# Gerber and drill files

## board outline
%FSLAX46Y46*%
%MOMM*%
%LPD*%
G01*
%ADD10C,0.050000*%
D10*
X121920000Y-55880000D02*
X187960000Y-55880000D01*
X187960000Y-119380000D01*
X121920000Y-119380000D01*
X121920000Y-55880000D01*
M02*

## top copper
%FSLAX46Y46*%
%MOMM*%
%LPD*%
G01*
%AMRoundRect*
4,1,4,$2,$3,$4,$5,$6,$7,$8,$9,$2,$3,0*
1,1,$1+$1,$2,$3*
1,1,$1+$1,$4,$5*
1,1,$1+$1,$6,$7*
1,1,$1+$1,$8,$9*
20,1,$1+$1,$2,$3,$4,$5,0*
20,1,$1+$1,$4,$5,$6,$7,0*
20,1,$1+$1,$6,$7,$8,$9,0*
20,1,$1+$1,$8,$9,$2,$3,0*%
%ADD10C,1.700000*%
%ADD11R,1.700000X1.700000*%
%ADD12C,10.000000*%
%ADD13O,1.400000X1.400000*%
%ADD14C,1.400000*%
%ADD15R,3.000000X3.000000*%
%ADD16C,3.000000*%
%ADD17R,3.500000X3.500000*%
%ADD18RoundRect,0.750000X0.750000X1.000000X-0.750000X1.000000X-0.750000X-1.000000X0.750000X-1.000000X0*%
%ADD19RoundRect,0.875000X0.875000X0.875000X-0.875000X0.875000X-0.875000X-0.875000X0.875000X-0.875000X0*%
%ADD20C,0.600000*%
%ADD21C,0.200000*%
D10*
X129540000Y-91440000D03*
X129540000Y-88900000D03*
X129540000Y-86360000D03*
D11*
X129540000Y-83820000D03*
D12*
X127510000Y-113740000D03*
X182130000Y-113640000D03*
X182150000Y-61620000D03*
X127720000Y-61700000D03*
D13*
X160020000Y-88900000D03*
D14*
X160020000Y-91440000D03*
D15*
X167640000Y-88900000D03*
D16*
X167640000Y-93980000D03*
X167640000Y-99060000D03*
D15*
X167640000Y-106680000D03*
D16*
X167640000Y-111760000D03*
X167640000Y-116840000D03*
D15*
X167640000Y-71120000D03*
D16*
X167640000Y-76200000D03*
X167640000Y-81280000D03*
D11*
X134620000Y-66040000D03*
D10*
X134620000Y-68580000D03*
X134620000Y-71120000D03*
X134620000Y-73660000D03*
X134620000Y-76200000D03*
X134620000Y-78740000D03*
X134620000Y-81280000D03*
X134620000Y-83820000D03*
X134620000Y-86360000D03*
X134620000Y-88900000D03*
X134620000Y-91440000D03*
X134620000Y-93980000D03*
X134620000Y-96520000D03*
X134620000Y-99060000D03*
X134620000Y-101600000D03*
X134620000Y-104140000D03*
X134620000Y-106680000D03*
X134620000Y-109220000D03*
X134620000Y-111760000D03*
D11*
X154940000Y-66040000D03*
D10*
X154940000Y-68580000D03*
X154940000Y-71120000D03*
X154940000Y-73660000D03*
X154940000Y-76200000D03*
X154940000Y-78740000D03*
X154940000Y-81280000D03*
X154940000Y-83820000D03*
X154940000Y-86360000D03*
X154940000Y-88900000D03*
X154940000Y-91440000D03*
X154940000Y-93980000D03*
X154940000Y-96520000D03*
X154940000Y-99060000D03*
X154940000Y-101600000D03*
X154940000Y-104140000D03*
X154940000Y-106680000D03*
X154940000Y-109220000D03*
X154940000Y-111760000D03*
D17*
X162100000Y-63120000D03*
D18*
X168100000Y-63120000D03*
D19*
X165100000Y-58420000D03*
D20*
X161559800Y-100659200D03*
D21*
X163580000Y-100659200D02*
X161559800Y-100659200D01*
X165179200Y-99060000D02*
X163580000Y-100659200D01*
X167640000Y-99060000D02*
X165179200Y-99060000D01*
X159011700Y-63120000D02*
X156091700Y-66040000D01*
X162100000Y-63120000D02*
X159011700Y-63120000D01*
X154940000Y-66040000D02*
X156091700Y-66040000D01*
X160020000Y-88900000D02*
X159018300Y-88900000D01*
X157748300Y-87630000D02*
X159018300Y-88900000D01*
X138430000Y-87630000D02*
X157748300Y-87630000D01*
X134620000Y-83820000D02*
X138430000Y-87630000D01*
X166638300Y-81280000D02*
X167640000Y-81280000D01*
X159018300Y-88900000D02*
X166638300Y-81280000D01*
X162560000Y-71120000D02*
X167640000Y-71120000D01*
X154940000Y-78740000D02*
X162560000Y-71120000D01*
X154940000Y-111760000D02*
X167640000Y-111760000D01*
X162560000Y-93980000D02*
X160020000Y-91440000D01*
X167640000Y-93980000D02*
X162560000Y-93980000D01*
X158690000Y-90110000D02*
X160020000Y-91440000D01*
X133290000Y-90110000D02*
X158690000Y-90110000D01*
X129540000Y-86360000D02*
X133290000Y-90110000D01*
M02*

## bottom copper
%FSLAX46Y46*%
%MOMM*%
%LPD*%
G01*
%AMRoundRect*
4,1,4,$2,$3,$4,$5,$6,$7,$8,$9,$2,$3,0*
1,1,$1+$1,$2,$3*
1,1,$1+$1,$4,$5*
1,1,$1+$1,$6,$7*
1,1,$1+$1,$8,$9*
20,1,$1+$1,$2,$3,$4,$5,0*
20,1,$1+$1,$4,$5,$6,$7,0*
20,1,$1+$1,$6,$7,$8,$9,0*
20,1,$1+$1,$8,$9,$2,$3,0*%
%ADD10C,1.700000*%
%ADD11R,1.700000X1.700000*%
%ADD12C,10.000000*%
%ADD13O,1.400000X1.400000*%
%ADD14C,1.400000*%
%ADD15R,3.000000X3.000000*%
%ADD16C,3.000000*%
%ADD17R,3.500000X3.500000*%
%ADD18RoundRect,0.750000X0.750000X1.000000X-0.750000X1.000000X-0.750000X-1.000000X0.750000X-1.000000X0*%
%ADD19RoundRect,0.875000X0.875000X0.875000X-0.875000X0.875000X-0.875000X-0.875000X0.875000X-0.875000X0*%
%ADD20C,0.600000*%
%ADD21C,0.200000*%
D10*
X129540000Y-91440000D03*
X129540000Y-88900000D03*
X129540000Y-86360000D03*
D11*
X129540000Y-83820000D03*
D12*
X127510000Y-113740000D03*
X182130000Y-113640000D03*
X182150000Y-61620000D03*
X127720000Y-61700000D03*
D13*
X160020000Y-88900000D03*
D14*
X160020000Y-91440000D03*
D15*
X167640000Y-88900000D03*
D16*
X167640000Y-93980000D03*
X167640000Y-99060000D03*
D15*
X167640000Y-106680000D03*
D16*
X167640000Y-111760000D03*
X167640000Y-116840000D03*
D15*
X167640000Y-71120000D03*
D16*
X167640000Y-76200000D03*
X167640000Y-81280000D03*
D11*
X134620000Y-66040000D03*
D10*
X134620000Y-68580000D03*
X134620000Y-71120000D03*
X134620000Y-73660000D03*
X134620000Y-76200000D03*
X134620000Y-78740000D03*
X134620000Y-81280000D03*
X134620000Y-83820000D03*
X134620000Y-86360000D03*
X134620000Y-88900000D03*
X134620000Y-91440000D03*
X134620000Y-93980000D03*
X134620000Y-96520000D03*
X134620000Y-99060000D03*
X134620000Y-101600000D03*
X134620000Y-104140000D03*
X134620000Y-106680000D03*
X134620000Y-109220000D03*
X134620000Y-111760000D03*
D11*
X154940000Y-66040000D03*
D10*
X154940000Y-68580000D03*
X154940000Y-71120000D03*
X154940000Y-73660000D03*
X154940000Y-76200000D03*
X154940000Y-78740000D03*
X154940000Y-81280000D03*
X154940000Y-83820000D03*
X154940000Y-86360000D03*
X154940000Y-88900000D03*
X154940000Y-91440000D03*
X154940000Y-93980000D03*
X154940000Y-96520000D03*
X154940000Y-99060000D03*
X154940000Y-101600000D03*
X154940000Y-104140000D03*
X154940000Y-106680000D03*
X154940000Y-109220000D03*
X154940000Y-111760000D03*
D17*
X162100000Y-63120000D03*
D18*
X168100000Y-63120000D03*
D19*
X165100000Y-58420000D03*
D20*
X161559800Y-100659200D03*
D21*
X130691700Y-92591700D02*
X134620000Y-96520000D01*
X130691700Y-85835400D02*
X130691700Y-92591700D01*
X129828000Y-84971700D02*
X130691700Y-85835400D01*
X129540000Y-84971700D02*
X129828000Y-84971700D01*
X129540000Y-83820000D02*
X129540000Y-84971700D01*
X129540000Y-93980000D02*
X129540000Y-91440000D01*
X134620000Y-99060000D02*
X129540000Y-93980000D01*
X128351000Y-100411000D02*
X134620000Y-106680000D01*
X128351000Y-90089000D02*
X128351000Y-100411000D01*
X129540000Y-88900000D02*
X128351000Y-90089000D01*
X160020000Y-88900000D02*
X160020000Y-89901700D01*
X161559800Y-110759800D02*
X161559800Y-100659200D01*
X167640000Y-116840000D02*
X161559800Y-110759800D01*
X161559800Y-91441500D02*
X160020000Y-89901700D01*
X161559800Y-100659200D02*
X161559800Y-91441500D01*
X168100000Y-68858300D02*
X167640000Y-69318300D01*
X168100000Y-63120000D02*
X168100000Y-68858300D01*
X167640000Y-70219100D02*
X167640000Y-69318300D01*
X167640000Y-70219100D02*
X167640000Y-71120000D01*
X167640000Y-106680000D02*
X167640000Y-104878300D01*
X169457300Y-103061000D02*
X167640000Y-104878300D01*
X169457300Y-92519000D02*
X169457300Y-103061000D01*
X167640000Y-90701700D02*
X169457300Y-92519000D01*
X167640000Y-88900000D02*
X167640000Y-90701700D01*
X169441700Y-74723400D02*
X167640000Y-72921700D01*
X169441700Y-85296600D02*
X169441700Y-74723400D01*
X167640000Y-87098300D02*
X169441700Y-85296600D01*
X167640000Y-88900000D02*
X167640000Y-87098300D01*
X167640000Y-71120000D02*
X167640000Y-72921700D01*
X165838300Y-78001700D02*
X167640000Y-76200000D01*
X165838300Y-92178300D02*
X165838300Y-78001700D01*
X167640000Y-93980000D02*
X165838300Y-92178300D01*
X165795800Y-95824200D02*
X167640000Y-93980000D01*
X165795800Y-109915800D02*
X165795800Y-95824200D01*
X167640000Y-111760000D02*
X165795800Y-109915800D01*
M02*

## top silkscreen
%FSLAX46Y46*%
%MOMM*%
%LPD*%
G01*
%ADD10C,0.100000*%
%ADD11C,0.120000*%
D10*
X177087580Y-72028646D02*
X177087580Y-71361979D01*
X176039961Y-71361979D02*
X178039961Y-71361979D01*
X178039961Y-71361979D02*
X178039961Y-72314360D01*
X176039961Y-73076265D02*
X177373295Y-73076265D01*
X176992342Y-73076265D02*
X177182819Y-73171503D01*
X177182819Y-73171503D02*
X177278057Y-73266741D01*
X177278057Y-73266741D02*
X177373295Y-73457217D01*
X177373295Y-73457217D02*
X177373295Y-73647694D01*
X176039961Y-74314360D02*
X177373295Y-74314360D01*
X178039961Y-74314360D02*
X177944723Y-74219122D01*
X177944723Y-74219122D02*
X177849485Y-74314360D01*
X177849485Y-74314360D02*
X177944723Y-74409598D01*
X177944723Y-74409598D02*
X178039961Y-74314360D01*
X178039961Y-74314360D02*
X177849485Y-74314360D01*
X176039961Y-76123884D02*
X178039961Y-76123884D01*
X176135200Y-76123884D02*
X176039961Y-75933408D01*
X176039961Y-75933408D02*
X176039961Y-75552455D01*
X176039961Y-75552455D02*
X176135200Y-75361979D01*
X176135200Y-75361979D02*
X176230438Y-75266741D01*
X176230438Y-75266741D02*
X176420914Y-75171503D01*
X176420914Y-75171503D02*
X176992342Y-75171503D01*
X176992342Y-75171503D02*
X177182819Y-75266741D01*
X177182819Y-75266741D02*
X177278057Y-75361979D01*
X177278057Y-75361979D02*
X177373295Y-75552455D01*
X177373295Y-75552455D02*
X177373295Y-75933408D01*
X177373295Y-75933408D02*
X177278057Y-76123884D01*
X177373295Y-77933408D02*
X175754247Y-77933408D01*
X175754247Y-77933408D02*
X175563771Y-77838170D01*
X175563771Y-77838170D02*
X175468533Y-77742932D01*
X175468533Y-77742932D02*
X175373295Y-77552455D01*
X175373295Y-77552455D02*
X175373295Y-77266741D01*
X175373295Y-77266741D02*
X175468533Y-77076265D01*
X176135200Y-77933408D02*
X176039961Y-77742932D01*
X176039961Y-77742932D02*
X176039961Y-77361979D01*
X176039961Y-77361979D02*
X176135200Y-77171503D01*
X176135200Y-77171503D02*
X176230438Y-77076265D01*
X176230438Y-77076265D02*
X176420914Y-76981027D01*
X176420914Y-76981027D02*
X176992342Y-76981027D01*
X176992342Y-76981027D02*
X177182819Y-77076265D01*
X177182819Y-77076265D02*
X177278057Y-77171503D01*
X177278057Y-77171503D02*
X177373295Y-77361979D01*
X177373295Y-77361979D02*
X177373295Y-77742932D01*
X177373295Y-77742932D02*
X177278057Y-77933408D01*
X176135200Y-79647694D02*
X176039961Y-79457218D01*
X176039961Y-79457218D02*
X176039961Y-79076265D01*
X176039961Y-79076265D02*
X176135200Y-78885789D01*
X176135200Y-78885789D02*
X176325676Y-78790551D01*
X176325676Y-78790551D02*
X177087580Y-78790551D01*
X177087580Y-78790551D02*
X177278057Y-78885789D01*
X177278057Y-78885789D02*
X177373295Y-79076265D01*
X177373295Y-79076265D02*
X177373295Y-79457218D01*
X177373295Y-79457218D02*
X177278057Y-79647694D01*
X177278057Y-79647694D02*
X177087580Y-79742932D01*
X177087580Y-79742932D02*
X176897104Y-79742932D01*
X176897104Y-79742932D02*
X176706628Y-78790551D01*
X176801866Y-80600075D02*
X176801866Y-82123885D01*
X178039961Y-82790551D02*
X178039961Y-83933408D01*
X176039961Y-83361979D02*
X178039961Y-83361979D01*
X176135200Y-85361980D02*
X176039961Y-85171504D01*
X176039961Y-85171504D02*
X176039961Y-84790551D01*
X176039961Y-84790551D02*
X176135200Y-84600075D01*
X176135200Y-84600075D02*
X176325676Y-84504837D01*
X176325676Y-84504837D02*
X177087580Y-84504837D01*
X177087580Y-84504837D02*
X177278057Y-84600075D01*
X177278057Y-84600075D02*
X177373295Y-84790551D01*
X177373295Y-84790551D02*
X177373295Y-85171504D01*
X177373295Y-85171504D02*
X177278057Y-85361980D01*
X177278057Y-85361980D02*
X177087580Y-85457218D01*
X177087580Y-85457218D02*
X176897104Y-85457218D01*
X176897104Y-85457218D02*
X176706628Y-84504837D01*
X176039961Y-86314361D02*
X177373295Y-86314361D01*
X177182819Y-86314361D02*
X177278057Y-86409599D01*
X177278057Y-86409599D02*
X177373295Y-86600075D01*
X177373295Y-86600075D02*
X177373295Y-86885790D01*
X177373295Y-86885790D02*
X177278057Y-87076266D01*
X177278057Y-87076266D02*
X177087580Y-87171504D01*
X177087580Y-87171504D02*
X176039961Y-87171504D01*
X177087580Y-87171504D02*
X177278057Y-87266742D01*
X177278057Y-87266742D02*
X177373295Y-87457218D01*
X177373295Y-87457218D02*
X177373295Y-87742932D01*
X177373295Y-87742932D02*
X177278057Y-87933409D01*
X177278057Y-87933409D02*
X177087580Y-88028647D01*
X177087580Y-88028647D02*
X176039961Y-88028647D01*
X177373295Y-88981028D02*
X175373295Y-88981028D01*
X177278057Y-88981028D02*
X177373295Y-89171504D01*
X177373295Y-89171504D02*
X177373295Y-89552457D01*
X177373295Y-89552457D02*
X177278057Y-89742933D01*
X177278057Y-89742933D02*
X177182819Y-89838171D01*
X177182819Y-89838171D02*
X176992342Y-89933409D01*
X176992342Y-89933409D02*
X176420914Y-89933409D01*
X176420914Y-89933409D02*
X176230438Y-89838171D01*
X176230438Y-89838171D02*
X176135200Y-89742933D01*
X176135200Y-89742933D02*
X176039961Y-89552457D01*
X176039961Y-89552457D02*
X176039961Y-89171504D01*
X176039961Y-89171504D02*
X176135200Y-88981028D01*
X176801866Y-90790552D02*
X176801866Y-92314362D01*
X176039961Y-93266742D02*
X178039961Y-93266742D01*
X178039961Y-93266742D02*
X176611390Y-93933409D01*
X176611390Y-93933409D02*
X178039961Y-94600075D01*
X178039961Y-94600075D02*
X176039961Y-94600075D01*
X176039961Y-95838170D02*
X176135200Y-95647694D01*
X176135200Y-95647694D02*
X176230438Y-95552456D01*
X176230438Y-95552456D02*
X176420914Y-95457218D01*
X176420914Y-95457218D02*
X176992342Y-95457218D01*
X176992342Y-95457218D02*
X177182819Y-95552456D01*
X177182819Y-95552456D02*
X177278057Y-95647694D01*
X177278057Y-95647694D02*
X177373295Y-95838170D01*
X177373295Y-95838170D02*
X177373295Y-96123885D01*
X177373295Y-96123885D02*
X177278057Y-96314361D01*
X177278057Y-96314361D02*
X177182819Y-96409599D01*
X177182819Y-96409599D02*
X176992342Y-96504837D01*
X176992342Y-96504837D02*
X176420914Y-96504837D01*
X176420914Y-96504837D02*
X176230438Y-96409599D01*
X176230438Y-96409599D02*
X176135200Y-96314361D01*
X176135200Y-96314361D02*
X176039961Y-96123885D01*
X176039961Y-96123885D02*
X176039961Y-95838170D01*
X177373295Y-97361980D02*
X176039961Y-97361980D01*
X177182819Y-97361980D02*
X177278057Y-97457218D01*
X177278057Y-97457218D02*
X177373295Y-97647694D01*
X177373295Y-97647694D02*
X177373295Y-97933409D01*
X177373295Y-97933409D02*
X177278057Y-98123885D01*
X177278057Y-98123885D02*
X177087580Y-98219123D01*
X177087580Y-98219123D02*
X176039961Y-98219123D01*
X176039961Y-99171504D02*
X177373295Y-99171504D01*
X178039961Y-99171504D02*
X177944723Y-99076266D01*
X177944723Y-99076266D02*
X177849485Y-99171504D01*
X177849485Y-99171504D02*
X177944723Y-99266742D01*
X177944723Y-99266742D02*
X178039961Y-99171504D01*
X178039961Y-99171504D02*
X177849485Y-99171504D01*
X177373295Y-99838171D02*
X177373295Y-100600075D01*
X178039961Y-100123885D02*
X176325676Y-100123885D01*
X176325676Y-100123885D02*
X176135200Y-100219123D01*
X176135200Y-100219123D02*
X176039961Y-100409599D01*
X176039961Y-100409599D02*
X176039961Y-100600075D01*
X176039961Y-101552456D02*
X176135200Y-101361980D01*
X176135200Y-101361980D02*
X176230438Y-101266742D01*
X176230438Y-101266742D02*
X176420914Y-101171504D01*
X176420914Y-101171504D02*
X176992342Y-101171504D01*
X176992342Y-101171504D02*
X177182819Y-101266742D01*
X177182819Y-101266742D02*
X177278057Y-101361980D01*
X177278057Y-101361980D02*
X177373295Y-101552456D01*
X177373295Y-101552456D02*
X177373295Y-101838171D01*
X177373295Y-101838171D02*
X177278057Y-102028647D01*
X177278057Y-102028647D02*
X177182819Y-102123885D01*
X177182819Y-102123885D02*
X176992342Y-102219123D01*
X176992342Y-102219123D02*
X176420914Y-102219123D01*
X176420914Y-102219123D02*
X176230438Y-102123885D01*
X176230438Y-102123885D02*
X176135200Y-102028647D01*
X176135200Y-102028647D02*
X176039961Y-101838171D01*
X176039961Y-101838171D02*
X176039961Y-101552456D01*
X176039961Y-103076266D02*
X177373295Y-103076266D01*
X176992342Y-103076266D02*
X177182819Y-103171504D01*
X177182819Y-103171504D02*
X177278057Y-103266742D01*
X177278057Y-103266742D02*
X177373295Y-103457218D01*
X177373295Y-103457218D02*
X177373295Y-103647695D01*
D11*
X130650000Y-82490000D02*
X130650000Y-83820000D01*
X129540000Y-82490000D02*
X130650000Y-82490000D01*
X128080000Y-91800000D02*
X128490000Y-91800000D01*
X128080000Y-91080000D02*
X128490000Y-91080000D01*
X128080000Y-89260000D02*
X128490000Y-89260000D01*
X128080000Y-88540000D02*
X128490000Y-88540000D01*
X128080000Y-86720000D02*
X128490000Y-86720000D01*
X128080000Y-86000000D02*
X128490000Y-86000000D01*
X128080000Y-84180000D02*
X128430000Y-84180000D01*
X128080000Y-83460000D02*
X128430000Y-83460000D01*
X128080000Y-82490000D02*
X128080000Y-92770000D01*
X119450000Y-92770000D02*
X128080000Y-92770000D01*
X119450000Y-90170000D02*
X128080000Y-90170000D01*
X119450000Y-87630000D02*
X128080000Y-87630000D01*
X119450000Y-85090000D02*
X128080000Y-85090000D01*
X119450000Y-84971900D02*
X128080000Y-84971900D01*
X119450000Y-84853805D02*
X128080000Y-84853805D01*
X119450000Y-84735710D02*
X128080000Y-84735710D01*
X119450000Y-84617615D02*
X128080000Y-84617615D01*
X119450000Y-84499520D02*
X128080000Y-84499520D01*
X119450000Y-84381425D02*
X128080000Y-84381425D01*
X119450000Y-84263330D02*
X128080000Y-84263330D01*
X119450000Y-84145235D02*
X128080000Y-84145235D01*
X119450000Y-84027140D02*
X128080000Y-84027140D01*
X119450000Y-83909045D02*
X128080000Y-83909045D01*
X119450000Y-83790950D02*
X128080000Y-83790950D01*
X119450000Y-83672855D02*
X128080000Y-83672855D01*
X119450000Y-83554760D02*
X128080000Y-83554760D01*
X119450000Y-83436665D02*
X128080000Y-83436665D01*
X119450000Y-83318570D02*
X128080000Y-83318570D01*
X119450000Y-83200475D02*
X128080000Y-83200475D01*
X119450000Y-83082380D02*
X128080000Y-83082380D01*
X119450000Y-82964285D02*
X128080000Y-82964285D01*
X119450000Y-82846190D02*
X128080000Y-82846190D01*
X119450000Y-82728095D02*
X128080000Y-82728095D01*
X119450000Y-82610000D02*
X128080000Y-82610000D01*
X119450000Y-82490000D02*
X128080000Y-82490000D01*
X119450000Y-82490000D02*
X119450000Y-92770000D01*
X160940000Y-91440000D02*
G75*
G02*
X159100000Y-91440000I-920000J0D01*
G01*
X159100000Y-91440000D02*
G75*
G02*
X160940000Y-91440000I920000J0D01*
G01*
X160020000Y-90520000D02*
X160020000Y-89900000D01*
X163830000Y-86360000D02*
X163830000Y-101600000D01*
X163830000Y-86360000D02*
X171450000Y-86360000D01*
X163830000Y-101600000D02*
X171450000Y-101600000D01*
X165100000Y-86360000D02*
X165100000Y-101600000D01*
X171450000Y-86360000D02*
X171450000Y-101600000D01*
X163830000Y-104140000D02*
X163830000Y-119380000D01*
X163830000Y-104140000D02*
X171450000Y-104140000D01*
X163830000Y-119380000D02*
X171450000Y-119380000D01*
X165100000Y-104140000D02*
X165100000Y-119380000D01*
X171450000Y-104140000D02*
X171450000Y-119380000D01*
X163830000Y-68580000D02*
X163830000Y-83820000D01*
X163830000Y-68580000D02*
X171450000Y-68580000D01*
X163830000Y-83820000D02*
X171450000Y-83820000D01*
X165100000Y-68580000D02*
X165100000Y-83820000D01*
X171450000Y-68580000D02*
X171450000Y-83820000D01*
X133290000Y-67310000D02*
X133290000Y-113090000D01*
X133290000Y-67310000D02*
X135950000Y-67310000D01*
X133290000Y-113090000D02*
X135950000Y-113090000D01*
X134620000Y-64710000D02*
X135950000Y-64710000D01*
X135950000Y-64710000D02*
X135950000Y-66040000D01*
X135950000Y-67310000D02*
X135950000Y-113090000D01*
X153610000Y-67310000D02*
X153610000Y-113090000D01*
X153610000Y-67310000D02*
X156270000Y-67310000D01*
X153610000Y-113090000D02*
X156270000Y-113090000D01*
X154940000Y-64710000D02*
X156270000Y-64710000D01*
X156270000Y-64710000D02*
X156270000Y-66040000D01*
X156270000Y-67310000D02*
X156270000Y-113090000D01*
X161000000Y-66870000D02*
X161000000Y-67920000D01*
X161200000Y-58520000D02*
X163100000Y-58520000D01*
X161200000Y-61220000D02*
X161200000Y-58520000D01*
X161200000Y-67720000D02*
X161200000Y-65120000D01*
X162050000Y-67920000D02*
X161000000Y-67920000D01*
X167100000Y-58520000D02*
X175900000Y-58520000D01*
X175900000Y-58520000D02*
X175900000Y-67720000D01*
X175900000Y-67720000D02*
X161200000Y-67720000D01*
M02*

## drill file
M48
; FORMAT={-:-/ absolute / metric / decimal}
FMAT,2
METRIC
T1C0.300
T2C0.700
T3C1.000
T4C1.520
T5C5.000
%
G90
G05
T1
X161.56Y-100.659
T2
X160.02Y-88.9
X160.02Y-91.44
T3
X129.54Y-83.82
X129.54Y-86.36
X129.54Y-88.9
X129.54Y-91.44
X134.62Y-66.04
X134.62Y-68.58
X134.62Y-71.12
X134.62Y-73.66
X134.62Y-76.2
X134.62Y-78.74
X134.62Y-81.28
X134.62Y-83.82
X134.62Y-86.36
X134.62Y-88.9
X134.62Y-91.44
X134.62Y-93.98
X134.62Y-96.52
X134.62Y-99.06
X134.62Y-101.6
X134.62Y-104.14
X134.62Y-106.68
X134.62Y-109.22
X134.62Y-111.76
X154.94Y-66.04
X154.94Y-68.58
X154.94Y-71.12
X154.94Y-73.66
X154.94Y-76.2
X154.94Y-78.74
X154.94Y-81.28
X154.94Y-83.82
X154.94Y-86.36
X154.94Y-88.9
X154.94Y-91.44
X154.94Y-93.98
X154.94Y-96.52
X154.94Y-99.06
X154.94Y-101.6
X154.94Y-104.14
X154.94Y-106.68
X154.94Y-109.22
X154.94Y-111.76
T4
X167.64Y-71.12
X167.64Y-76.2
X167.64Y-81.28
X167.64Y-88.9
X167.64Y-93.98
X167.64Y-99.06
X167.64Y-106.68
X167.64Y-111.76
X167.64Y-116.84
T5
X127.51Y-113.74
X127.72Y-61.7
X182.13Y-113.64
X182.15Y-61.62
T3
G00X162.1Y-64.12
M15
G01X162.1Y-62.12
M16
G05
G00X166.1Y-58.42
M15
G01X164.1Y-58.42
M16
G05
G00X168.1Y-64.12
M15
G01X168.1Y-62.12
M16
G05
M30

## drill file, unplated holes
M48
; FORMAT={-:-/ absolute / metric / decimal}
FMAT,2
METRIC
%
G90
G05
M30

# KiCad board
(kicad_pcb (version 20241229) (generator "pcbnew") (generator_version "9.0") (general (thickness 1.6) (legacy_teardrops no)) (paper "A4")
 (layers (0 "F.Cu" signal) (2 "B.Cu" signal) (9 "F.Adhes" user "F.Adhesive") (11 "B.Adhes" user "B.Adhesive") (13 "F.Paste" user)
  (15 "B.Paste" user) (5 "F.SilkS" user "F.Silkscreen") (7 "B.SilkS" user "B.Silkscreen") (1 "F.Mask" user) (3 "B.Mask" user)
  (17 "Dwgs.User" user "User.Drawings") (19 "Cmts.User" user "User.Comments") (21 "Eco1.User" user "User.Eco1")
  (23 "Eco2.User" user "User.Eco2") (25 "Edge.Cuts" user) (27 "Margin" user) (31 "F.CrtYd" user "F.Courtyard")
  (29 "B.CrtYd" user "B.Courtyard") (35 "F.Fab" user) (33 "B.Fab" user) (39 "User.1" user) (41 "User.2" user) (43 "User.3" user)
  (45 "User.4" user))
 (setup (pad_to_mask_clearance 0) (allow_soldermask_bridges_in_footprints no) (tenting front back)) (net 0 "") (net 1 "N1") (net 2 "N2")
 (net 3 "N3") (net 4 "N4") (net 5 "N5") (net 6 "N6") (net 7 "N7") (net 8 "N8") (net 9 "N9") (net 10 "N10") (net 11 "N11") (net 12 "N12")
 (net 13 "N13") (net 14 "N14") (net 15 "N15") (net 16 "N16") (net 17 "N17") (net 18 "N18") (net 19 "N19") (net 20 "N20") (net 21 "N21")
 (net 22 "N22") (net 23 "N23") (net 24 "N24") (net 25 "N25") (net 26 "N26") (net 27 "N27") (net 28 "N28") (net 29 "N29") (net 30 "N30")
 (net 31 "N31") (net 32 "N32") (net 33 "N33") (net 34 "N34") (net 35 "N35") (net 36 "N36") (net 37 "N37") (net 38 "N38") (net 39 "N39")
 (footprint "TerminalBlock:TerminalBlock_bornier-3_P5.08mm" (layer "F.Cu") (at 167.64 88.9 -90)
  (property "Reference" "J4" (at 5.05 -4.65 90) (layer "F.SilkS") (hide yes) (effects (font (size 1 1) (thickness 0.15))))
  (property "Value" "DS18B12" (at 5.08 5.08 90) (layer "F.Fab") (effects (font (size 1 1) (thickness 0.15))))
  (fp_line (start -2.54 3.81) (end 12.7 3.81) (stroke (width 0.12) (type solid)) (layer "F.SilkS"))
  (fp_line (start -2.54 3.81) (end -2.54 -3.81) (stroke (width 0.12) (type solid)) (layer "F.SilkS"))
  (fp_line (start 12.7 3.81) (end 12.7 -3.81) (stroke (width 0.12) (type solid)) (layer "F.SilkS"))
  (fp_line (start -2.54 2.54) (end 12.7 2.54) (stroke (width 0.12) (type solid)) (layer "F.SilkS"))
  (fp_line (start -2.54 -3.81) (end 12.7 -3.81) (stroke (width 0.12) (type solid)) (layer "F.SilkS"))
  (pad "1" thru_hole rect (at 0 0 270) (size 3 3) (drill 1.52) (layers "*.Cu" "*.Mask") (remove_unused_layers no) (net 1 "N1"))
  (pad "2" thru_hole circle (at 5.08 0 270) (size 3 3) (drill 1.52) (layers "*.Cu" "*.Mask") (remove_unused_layers no) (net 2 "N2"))
  (pad "3" thru_hole circle (at 10.16 0 270) (size 3 3) (drill 1.52) (layers "*.Cu" "*.Mask") (remove_unused_layers no) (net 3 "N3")))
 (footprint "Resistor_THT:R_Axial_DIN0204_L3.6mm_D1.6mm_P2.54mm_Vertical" (layer "F.Cu") (at 160.02 91.44 90)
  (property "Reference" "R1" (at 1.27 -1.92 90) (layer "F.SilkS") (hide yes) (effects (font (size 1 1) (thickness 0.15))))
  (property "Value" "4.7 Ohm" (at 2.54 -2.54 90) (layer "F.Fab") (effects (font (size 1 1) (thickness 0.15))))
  (fp_line (start 0.92 0) (end 1.54 0) (stroke (width 0.12) (type solid)) (layer "F.SilkS"))
  (fp_circle (center 0 0) (end 0.92 0) (stroke (width 0.12) (type solid)) (fill no) (layer "F.SilkS"))
  (pad "1" thru_hole circle (at 0 0 90) (size 1.4 1.4) (drill 0.7) (layers "*.Cu" "*.Mask") (remove_unused_layers no) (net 2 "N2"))
  (pad "2" thru_hole oval (at 2.54 0 90) (size 1.4 1.4) (drill 0.7) (layers "*.Cu" "*.Mask") (remove_unused_layers no) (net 3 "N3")))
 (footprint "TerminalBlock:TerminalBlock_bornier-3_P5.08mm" (layer "F.Cu") (at 167.64 106.68 -90)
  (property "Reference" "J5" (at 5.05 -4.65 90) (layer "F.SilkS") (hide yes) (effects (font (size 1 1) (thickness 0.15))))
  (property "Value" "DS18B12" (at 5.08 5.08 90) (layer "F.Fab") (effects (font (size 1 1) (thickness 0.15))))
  (fp_line (start -2.54 3.81) (end 12.7 3.81) (stroke (width 0.12) (type solid)) (layer "F.SilkS"))
  (fp_line (start -2.54 3.81) (end -2.54 -3.81) (stroke (width 0.12) (type solid)) (layer "F.SilkS"))
  (fp_line (start 12.7 3.81) (end 12.7 -3.81) (stroke (width 0.12) (type solid)) (layer "F.SilkS"))
  (fp_line (start -2.54 2.54) (end 12.7 2.54) (stroke (width 0.12) (type solid)) (layer "F.SilkS"))
  (fp_line (start -2.54 -3.81) (end 12.7 -3.81) (stroke (width 0.12) (type solid)) (layer "F.SilkS"))
  (pad "1" thru_hole rect (at 0 0 270) (size 3 3) (drill 1.52) (layers "*.Cu" "*.Mask") (remove_unused_layers no) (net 1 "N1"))
  (pad "2" thru_hole circle (at 5.08 0 270) (size 3 3) (drill 1.52) (layers "*.Cu" "*.Mask") (remove_unused_layers no) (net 2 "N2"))
  (pad "3" thru_hole circle (at 10.16 0 270) (size 3 3) (drill 1.52) (layers "*.Cu" "*.Mask") (remove_unused_layers no) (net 3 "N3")))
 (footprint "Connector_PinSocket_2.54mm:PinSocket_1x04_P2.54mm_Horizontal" (layer "F.Cu") (at 129.54 83.82)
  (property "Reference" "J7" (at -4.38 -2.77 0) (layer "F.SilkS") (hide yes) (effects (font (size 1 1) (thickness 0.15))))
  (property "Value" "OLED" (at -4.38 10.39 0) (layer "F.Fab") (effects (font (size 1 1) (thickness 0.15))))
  (fp_line (start -10.09 -1.33) (end -10.09 8.95) (stroke (width 0.12) (type solid)) (layer "F.SilkS"))
  (fp_line (start -10.09 -1.33) (end -1.46 -1.33) (stroke (width 0.12) (type solid)) (layer "F.SilkS"))
  (fp_line (start -10.09 -1.21) (end -1.46 -1.21) (stroke (width 0.12) (type solid)) (layer "F.SilkS"))
  (fp_line (start -10.09 -1.091905) (end -1.46 -1.091905) (stroke (width 0.12) (type solid)) (layer "F.SilkS"))
  (fp_line (start -10.09 -0.97381) (end -1.46 -0.97381) (stroke (width 0.12) (type solid)) (layer "F.SilkS"))
  (fp_line (start -10.09 -0.855715) (end -1.46 -0.855715) (stroke (width 0.12) (type solid)) (layer "F.SilkS"))
  (fp_line (start -10.09 -0.73762) (end -1.46 -0.73762) (stroke (width 0.12) (type solid)) (layer "F.SilkS"))
  (fp_line (start -10.09 -0.619525) (end -1.46 -0.619525) (stroke (width 0.12) (type solid)) (layer "F.SilkS"))
  (fp_line (start -10.09 -0.50143) (end -1.46 -0.50143) (stroke (width 0.12) (type solid)) (layer "F.SilkS"))
  (fp_line (start -10.09 -0.383335) (end -1.46 -0.383335) (stroke (width 0.12) (type solid)) (layer "F.SilkS"))
  (fp_line (start -10.09 -0.26524) (end -1.46 -0.26524) (stroke (width 0.12) (type solid)) (layer "F.SilkS"))
  (fp_line (start -10.09 -0.147145) (end -1.46 -0.147145) (stroke (width 0.12) (type solid)) (layer "F.SilkS"))
  (fp_line (start -10.09 -0.02905) (end -1.46 -0.02905) (stroke (width 0.12) (type solid)) (layer "F.SilkS"))
  (fp_line (start -10.09 0.089045) (end -1.46 0.089045) (stroke (width 0.12) (type solid)) (layer "F.SilkS"))
  (fp_line (start -10.09 0.20714) (end -1.46 0.20714) (stroke (width 0.12) (type solid)) (layer "F.SilkS"))
  (fp_line (start -10.09 0.325235) (end -1.46 0.325235) (stroke (width 0.12) (type solid)) (layer "F.SilkS"))
  (fp_line (start -10.09 0.44333) (end -1.46 0.44333) (stroke (width 0.12) (type solid)) (layer "F.SilkS"))
  (fp_line (start -10.09 0.561425) (end -1.46 0.561425) (stroke (width 0.12) (type solid)) (layer "F.SilkS"))
  (fp_line (start -10.09 0.67952) (end -1.46 0.67952) (stroke (width 0.12) (type solid)) (layer "F.SilkS"))
  (fp_line (start -10.09 0.797615) (end -1.46 0.797615) (stroke (width 0.12) (type solid)) (layer "F.SilkS"))
  (fp_line (start -10.09 0.91571) (end -1.46 0.91571) (stroke (width 0.12) (type solid)) (layer "F.SilkS"))
  (fp_line (start -10.09 1.033805) (end -1.46 1.033805) (stroke (width 0.12) (type solid)) (layer "F.SilkS"))
  (fp_line (start -10.09 1.1519) (end -1.46 1.1519) (stroke (width 0.12) (type solid)) (layer "F.SilkS"))
  (fp_line (start -10.09 1.27) (end -1.46 1.27) (stroke (width 0.12) (type solid)) (layer "F.SilkS"))
  (fp_line (start -10.09 3.81) (end -1.46 3.81) (stroke (width 0.12) (type solid)) (layer "F.SilkS"))
  (fp_line (start -10.09 6.35) (end -1.46 6.35) (stroke (width 0.12) (type solid)) (layer "F.SilkS"))
  (fp_line (start -10.09 8.95) (end -1.46 8.95) (stroke (width 0.12) (type solid)) (layer "F.SilkS"))
  (fp_line (start -1.46 -1.33) (end -1.46 8.95) (stroke (width 0.12) (type solid)) (layer "F.SilkS"))
  (fp_line (start -1.46 -0.36) (end -1.11 -0.36) (stroke (width 0.12) (type solid)) (layer "F.SilkS"))
  (fp_line (start -1.46 0.36) (end -1.11 0.36) (stroke (width 0.12) (type solid)) (layer "F.SilkS"))
  (fp_line (start -1.46 2.18) (end -1.05 2.18) (stroke (width 0.12) (type solid)) (layer "F.SilkS"))
  (fp_line (start -1.46 2.9) (end -1.05 2.9) (stroke (width 0.12) (type solid)) (layer "F.SilkS"))
  (fp_line (start -1.46 4.72) (end -1.05 4.72) (stroke (width 0.12) (type solid)) (layer "F.SilkS"))
  (fp_line (start -1.46 5.44) (end -1.05 5.44) (stroke (width 0.12) (type solid)) (layer "F.SilkS"))
  (fp_line (start -1.46 7.26) (end -1.05 7.26) (stroke (width 0.12) (type solid)) (layer "F.SilkS"))
  (fp_line (start -1.46 7.98) (end -1.05 7.98) (stroke (width 0.12) (type solid)) (layer "F.SilkS"))
  (fp_line (start 0 -1.33) (end 1.11 -1.33) (stroke (width 0.12) (type solid)) (layer "F.SilkS"))
  (fp_line (start 1.11 -1.33) (end 1.11 0) (stroke (width 0.12) (type solid)) (layer "F.SilkS"))
  (pad "1" thru_hole rect (at 0 0) (size 1.7 1.7) (drill 1) (layers "*.Cu" "*.Mask") (remove_unused_layers no) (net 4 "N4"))
  (pad "2" thru_hole circle (at 0 2.54) (size 1.7 1.7) (drill 1) (layers "*.Cu" "*.Mask") (remove_unused_layers no) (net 2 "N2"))
  (pad "3" thru_hole circle (at 0 5.08) (size 1.7 1.7) (drill 1) (layers "*.Cu" "*.Mask") (remove_unused_layers no) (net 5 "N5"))
  (pad "4" thru_hole circle (at 0 7.62) (size 1.7 1.7) (drill 1) (layers "*.Cu" "*.Mask") (remove_unused_layers no) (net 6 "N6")))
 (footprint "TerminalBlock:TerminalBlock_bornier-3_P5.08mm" (layer "F.Cu") (at 167.64 71.12 -90)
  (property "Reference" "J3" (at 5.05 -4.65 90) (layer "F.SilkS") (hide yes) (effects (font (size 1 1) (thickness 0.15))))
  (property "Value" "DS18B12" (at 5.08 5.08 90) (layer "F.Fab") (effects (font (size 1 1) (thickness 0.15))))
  (fp_line (start -2.54 3.81) (end 12.7 3.81) (stroke (width 0.12) (type solid)) (layer "F.SilkS"))
  (fp_line (start -2.54 3.81) (end -2.54 -3.81) (stroke (width 0.12) (type solid)) (layer "F.SilkS"))
  (fp_line (start 12.7 3.81) (end 12.7 -3.81) (stroke (width 0.12) (type solid)) (layer "F.SilkS"))
  (fp_line (start -2.54 2.54) (end 12.7 2.54) (stroke (width 0.12) (type solid)) (layer "F.SilkS"))
  (fp_line (start -2.54 -3.81) (end 12.7 -3.81) (stroke (width 0.12) (type solid)) (layer "F.SilkS"))
  (pad "1" thru_hole rect (at 0 0 270) (size 3 3) (drill 1.52) (layers "*.Cu" "*.Mask") (remove_unused_layers no) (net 1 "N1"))
  (pad "2" thru_hole circle (at 5.08 0 270) (size 3 3) (drill 1.52) (layers "*.Cu" "*.Mask") (remove_unused_layers no) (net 2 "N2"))
  (pad "3" thru_hole circle (at 10.16 0 270) (size 3 3) (drill 1.52) (layers "*.Cu" "*.Mask") (remove_unused_layers no) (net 3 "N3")))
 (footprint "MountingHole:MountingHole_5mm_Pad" (layer "F.Cu") (at 127.51 113.74)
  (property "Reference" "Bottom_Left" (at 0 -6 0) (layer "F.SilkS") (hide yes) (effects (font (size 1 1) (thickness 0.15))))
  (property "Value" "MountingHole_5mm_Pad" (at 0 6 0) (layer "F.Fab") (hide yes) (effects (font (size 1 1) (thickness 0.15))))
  (pad "1" thru_hole circle (at 0 0) (size 10 10) (drill 5) (layers "*.Cu" "*.Mask") (remove_unused_layers no)))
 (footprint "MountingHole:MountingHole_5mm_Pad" (layer "F.Cu") (at 182.15 61.62)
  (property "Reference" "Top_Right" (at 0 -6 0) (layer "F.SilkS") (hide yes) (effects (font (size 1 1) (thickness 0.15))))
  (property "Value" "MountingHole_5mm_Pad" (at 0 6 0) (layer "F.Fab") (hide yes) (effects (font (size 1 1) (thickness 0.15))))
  (pad "1" thru_hole circle (at 0 0) (size 10 10) (drill 5) (layers "*.Cu" "*.Mask") (remove_unused_layers no)))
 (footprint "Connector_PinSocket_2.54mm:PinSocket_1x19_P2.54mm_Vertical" (layer "F.Cu") (at 134.62 66.04)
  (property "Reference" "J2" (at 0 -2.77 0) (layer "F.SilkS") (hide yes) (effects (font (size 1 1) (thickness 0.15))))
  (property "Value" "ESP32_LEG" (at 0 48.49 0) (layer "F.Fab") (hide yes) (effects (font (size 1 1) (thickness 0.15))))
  (fp_line (start -1.33 1.27) (end -1.33 47.05) (stroke (width 0.12) (type solid)) (layer "F.SilkS"))
  (fp_line (start -1.33 1.27) (end 1.33 1.27) (stroke (width 0.12) (type solid)) (layer "F.SilkS"))
  (fp_line (start -1.33 47.05) (end 1.33 47.05) (stroke (width 0.12) (type solid)) (layer "F.SilkS"))
  (fp_line (start 0 -1.33) (end 1.33 -1.33) (stroke (width 0.12) (type solid)) (layer "F.SilkS"))
  (fp_line (start 1.33 -1.33) (end 1.33 0) (stroke (width 0.12) (type solid)) (layer "F.SilkS"))
  (fp_line (start 1.33 1.27) (end 1.33 47.05) (stroke (width 0.12) (type solid)) (layer "F.SilkS"))
  (pad "1" thru_hole rect (at 0 0) (size 1.7 1.7) (drill 1) (layers "*.Cu" "*.Mask") (remove_unused_layers no) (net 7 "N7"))
  (pad "2" thru_hole circle (at 0 2.54) (size 1.7 1.7) (drill 1) (layers "*.Cu" "*.Mask") (remove_unused_layers no) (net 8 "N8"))
  (pad "3" thru_hole circle (at 0 5.08) (size 1.7 1.7) (drill 1) (layers "*.Cu" "*.Mask") (remove_unused_layers no) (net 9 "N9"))
  (pad "4" thru_hole circle (at 0 7.62) (size 1.7 1.7) (drill 1) (layers "*.Cu" "*.Mask") (remove_unused_layers no) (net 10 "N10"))
  (pad "5" thru_hole circle (at 0 10.16) (size 1.7 1.7) (drill 1) (layers "*.Cu" "*.Mask") (remove_unused_layers no) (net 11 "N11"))
  (pad "6" thru_hole circle (at 0 12.7) (size 1.7 1.7) (drill 1) (layers "*.Cu" "*.Mask") (remove_unused_layers no) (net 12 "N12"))
  (pad "7" thru_hole circle (at 0 15.24) (size 1.7 1.7) (drill 1) (layers "*.Cu" "*.Mask") (remove_unused_layers no) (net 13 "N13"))
  (pad "8" thru_hole circle (at 0 17.78) (size 1.7 1.7) (drill 1) (layers "*.Cu" "*.Mask") (remove_unused_layers no) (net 3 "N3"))
  (pad "9" thru_hole circle (at 0 20.32) (size 1.7 1.7) (drill 1) (layers "*.Cu" "*.Mask") (remove_unused_layers no) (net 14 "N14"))
  (pad "10" thru_hole circle (at 0 22.86) (size 1.7 1.7) (drill 1) (layers "*.Cu" "*.Mask") (remove_unused_layers no) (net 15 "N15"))
  (pad "11" thru_hole circle (at 0 25.4) (size 1.7 1.7) (drill 1) (layers "*.Cu" "*.Mask") (remove_unused_layers no) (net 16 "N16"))
  (pad "12" thru_hole circle (at 0 27.94) (size 1.7 1.7) (drill 1) (layers "*.Cu" "*.Mask") (remove_unused_layers no) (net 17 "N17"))
  (pad "13" thru_hole circle (at 0 30.48) (size 1.7 1.7) (drill 1) (layers "*.Cu" "*.Mask") (remove_unused_layers no) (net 4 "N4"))
  (pad "14" thru_hole circle (at 0 33.02) (size 1.7 1.7) (drill 1) (layers "*.Cu" "*.Mask") (remove_unused_layers no) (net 6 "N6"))
  (pad "15" thru_hole circle (at 0 35.56) (size 1.7 1.7) (drill 1) (layers "*.Cu" "*.Mask") (remove_unused_layers no) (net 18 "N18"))
  (pad "16" thru_hole circle (at 0 38.1) (size 1.7 1.7) (drill 1) (layers "*.Cu" "*.Mask") (remove_unused_layers no) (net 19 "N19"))
  (pad "17" thru_hole circle (at 0 40.64) (size 1.7 1.7) (drill 1) (layers "*.Cu" "*.Mask") (remove_unused_layers no) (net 5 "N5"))
  (pad "18" thru_hole circle (at 0 43.18) (size 1.7 1.7) (drill 1) (layers "*.Cu" "*.Mask") (remove_unused_layers no) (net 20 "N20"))
  (pad "19" thru_hole circle (at 0 45.72) (size 1.7 1.7) (drill 1) (layers "*.Cu" "*.Mask") (remove_unused_layers no) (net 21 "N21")))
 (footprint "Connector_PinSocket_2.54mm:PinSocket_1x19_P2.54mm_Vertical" (layer "F.Cu") (at 154.94 66.04)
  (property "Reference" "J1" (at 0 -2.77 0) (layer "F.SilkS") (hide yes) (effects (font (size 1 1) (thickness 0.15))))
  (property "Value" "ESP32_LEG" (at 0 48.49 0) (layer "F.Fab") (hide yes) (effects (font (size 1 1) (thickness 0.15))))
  (fp_line (start -1.33 1.27) (end -1.33 47.05) (stroke (width 0.12) (type solid)) (layer "F.SilkS"))
  (fp_line (start -1.33 1.27) (end 1.33 1.27) (stroke (width 0.12) (type solid)) (layer "F.SilkS"))
  (fp_line (start -1.33 47.05) (end 1.33 47.05) (stroke (width 0.12) (type solid)) (layer "F.SilkS"))
  (fp_line (start 0 -1.33) (end 1.33 -1.33) (stroke (width 0.12) (type solid)) (layer "F.SilkS"))
  (fp_line (start 1.33 -1.33) (end 1.33 0) (stroke (width 0.12) (type solid)) (layer "F.SilkS"))
  (fp_line (start 1.33 1.27) (end 1.33 47.05) (stroke (width 0.12) (type solid)) (layer "F.SilkS"))
  (pad "1" thru_hole rect (at 0 0) (size 1.7 1.7) (drill 1) (layers "*.Cu" "*.Mask") (remove_unused_layers no) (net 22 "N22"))
  (pad "2" thru_hole circle (at 0 2.54) (size 1.7 1.7) (drill 1) (layers "*.Cu" "*.Mask") (remove_unused_layers no) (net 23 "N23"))
  (pad "3" thru_hole circle (at 0 5.08) (size 1.7 1.7) (drill 1) (layers "*.Cu" "*.Mask") (remove_unused_layers no) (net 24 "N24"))
  (pad "4" thru_hole circle (at 0 7.62) (size 1.7 1.7) (drill 1) (layers "*.Cu" "*.Mask") (remove_unused_layers no) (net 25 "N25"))
  (pad "5" thru_hole circle (at 0 10.16) (size 1.7 1.7) (drill 1) (layers "*.Cu" "*.Mask") (remove_unused_layers no) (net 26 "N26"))
  (pad "6" thru_hole circle (at 0 12.7) (size 1.7 1.7) (drill 1) (layers "*.Cu" "*.Mask") (remove_unused_layers no) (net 1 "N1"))
  (pad "7" thru_hole circle (at 0 15.24) (size 1.7 1.7) (drill 1) (layers "*.Cu" "*.Mask") (remove_unused_layers no) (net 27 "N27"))
  (pad "8" thru_hole circle (at 0 17.78) (size 1.7 1.7) (drill 1) (layers "*.Cu" "*.Mask") (remove_unused_layers no) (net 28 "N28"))
  (pad "9" thru_hole circle (at 0 20.32) (size 1.7 1.7) (drill 1) (layers "*.Cu" "*.Mask") (remove_unused_layers no) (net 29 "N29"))
  (pad "10" thru_hole circle (at 0 22.86) (size 1.7 1.7) (drill 1) (layers "*.Cu" "*.Mask") (remove_unused_layers no) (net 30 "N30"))
  (pad "11" thru_hole circle (at 0 25.4) (size 1.7 1.7) (drill 1) (layers "*.Cu" "*.Mask") (remove_unused_layers no) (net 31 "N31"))
  (pad "12" thru_hole circle (at 0 27.94) (size 1.7 1.7) (drill 1) (layers "*.Cu" "*.Mask") (remove_unused_layers no) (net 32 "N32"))
  (pad "13" thru_hole circle (at 0 30.48) (size 1.7 1.7) (drill 1) (layers "*.Cu" "*.Mask") (remove_unused_layers no) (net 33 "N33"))
  (pad "14" thru_hole circle (at 0 33.02) (size 1.7 1.7) (drill 1) (layers "*.Cu" "*.Mask") (remove_unused_layers no) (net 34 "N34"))
  (pad "15" thru_hole circle (at 0 35.56) (size 1.7 1.7) (drill 1) (layers "*.Cu" "*.Mask") (remove_unused_layers no) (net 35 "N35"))
  (pad "16" thru_hole circle (at 0 38.1) (size 1.7 1.7) (drill 1) (layers "*.Cu" "*.Mask") (remove_unused_layers no) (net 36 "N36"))
  (pad "17" thru_hole circle (at 0 40.64) (size 1.7 1.7) (drill 1) (layers "*.Cu" "*.Mask") (remove_unused_layers no) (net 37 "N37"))
  (pad "18" thru_hole circle (at 0 43.18) (size 1.7 1.7) (drill 1) (layers "*.Cu" "*.Mask") (remove_unused_layers no) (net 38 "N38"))
  (pad "19" thru_hole circle (at 0 45.72) (size 1.7 1.7) (drill 1) (layers "*.Cu" "*.Mask") (remove_unused_layers no) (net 2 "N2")))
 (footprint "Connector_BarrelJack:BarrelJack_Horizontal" (layer "F.Cu") (at 162.1 63.12 180)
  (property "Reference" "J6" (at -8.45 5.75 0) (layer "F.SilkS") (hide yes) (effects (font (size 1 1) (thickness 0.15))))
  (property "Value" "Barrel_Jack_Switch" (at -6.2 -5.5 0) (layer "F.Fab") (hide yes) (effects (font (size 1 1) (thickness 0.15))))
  (fp_line (start 1.1 -3.75) (end 1.1 -4.8) (stroke (width 0.12) (type solid)) (layer "F.SilkS"))
  (fp_line (start 0.9 4.6) (end -1 4.6) (stroke (width 0.12) (type solid)) (layer "F.SilkS"))
  (fp_line (start 0.9 1.9) (end 0.9 4.6) (stroke (width 0.12) (type solid)) (layer "F.SilkS"))
  (fp_line (start 0.9 -4.6) (end 0.9 -2) (stroke (width 0.12) (type solid)) (layer "F.SilkS"))
  (fp_line (start 0.05 -4.8) (end 1.1 -4.8) (stroke (width 0.12) (type solid)) (layer "F.SilkS"))
  (fp_line (start -5 4.6) (end -13.8 4.6) (stroke (width 0.12) (type solid)) (layer "F.SilkS"))
  (fp_line (start -13.8 4.6) (end -13.8 -4.6) (stroke (width 0.12) (type solid)) (layer "F.SilkS"))
  (fp_line (start -13.8 -4.6) (end 0.9 -4.6) (stroke (width 0.12) (type solid)) (layer "F.SilkS"))
  (pad "1" thru_hole rect (at 0 0 180) (size 3.5 3.5) (drill oval 1 3) (layers "*.Cu" "*.Mask") (remove_unused_layers no) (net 22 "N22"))
  (pad "2" thru_hole roundrect (at -6 0 180) (size 3 3.5) (drill oval 1 3) (layers "*.Cu" "*.Mask") (remove_unused_layers no)
   (roundrect_rratio 0.25) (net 1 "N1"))
  (pad "3" thru_hole roundrect (at -3 4.7 180) (size 3.5 3.5) (drill oval 3 1) (layers "*.Cu" "*.Mask") (remove_unused_layers no)
   (roundrect_rratio 0.25) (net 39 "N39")))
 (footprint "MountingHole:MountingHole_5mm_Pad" (layer "F.Cu") (at 182.13 113.64)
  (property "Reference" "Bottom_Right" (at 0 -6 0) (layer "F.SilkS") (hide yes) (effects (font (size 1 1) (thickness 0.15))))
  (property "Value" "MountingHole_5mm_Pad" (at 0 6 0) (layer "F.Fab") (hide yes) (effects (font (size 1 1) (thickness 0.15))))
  (pad "1" thru_hole circle (at 0 0) (size 10 10) (drill 5) (layers "*.Cu" "*.Mask") (remove_unused_layers no)))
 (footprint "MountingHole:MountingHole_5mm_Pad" (layer "F.Cu") (at 127.72 61.7)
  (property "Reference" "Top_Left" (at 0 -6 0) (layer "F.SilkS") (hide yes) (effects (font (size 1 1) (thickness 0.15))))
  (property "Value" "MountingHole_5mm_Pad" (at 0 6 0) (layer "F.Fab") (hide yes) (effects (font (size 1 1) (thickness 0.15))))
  (pad "1" thru_hole circle (at 0 0) (size 10 10) (drill 5) (layers "*.Cu" "*.Mask") (remove_unused_layers no)))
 (gr_rect (start 121.92 55.88) (end 187.96 119.38) (stroke (width 0.05) (type default)) (fill no) (layer "Edge.Cuts"))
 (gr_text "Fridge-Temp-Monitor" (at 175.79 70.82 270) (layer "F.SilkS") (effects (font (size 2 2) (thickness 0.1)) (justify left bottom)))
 (segment (start 162.56 93.98) (end 160.02 91.44) (width 0.2) (layer "F.Cu") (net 2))
 (segment (start 158.69 90.11) (end 160.02 91.44) (width 0.2) (layer "F.Cu") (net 2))
 (segment (start 133.29 90.11) (end 158.69 90.11) (width 0.2) (layer "F.Cu") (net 2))
 (segment (start 167.64 93.98) (end 162.56 93.98) (width 0.2) (layer "F.Cu") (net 2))
 (segment (start 129.54 86.36) (end 133.29 90.11) (width 0.2) (layer "F.Cu") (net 2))
 (segment (start 154.94 111.76) (end 167.64 111.76) (width 0.2) (layer "F.Cu") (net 2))
 (segment (start 165.7958 95.8242) (end 167.64 93.98) (width 0.2) (layer "B.Cu") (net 2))
 (segment (start 165.8383 78.0017) (end 167.64 76.2) (width 0.2) (layer "B.Cu") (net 2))
 (segment (start 165.7958 109.9158) (end 165.7958 95.8242) (width 0.2) (layer "B.Cu") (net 2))
 (segment (start 167.64 93.98) (end 165.8383 92.1783) (width 0.2) (layer "B.Cu") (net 2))
 (segment (start 165.8383 92.1783) (end 165.8383 78.0017) (width 0.2) (layer "B.Cu") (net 2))
 (segment (start 167.64 111.76) (end 165.7958 109.9158) (width 0.2) (layer "B.Cu") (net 2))
 (segment (start 162.56 71.12) (end 167.64 71.12) (width 0.2) (layer "F.Cu") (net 1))
 (segment (start 154.94 78.74) (end 162.56 71.12) (width 0.2) (layer "F.Cu") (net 1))
 (segment (start 167.64 70.2191) (end 167.64 69.3183) (width 0.2) (layer "B.Cu") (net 1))
 (segment (start 169.4417 85.2966) (end 169.4417 74.7234) (width 0.2) (layer "B.Cu") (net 1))
 (segment (start 167.64 88.9) (end 167.64 87.0983) (width 0.2) (layer "B.Cu") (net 1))
 (segment (start 169.4417 74.7234) (end 167.64 72.9217) (width 0.2) (layer "B.Cu") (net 1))
 (segment (start 167.64 70.2191) (end 167.64 71.12) (width 0.2) (layer "B.Cu") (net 1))
 (segment (start 167.64 88.9) (end 167.64 90.7017) (width 0.2) (layer "B.Cu") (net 1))
 (segment (start 169.4573 103.061) (end 167.64 104.8783) (width 0.2) (layer "B.Cu") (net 1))
 (segment (start 168.1 63.12) (end 168.1 68.8583) (width 0.2) (layer "B.Cu") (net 1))
 (segment (start 168.1 68.8583) (end 167.64 69.3183) (width 0.2) (layer "B.Cu") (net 1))
 (segment (start 167.64 87.0983) (end 169.4417 85.2966) (width 0.2) (layer "B.Cu") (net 1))
 (segment (start 167.64 71.12) (end 167.64 72.9217) (width 0.2) (layer "B.Cu") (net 1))
 (segment (start 167.64 106.68) (end 167.64 104.8783) (width 0.2) (layer "B.Cu") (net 1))
 (segment (start 167.64 90.7017) (end 169.4573 92.519) (width 0.2) (layer "B.Cu") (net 1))
 (segment (start 169.4573 92.519) (end 169.4573 103.061) (width 0.2) (layer "B.Cu") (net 1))
 (segment (start 163.58 100.6592) (end 161.5598 100.6592) (width 0.2) (layer "F.Cu") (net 3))
 (segment (start 159.0183 88.9) (end 166.6383 81.28) (width 0.2) (layer "F.Cu") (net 3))
 (segment (start 167.64 99.06) (end 165.1792 99.06) (width 0.2) (layer "F.Cu") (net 3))
 (segment (start 165.1792 99.06) (end 163.58 100.6592) (width 0.2) (layer "F.Cu") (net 3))
 (segment (start 134.62 83.82) (end 138.43 87.63) (width 0.2) (layer "F.Cu") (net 3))
 (segment (start 166.6383 81.28) (end 167.64 81.28) (width 0.2) (layer "F.Cu") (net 3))
 (segment (start 157.7483 87.63) (end 159.0183 88.9) (width 0.2) (layer "F.Cu") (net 3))
 (segment (start 160.02 88.9) (end 159.0183 88.9) (width 0.2) (layer "F.Cu") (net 3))
 (segment (start 138.43 87.63) (end 157.7483 87.63) (width 0.2) (layer "F.Cu") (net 3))
 (via (at 161.5598 100.6592) (size 0.6) (drill 0.3) (layers "F.Cu" "B.Cu") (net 3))
 (segment (start 167.64 116.84) (end 161.5598 110.7598) (width 0.2) (layer "B.Cu") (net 3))
 (segment (start 161.5598 91.4415) (end 160.02 89.9017) (width 0.2) (layer "B.Cu") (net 3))
 (segment (start 160.02 88.9) (end 160.02 89.9017) (width 0.2) (layer "B.Cu") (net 3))
 (segment (start 161.5598 100.6592) (end 161.5598 91.4415) (width 0.2) (layer "B.Cu") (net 3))
 (segment (start 161.5598 110.7598) (end 161.5598 100.6592) (width 0.2) (layer "B.Cu") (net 3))
 (segment (start 128.351 100.411) (end 134.62 106.68) (width 0.2) (layer "B.Cu") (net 5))
 (segment (start 128.351 90.089) (end 128.351 100.411) (width 0.2) (layer "B.Cu") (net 5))
 (segment (start 129.54 88.9) (end 128.351 90.089) (width 0.2) (layer "B.Cu") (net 5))
 (segment (start 134.62 99.06) (end 129.54 93.98) (width 0.2) (layer "B.Cu") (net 6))
 (segment (start 129.54 93.98) (end 129.54 91.44) (width 0.2) (layer "B.Cu") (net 6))
 (segment (start 129.828 84.9717) (end 130.6917 85.8354) (width 0.2) (layer "B.Cu") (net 4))
 (segment (start 129.54 84.9717) (end 129.828 84.9717) (width 0.2) (layer "B.Cu") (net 4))
 (segment (start 130.6917 92.5917) (end 134.62 96.52) (width 0.2) (layer "B.Cu") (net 4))
 (segment (start 130.6917 85.8354) (end 130.6917 92.5917) (width 0.2) (layer "B.Cu") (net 4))
 (segment (start 129.54 83.82) (end 129.54 84.9717) (width 0.2) (layer "B.Cu") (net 4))
 (segment (start 162.1 63.12) (end 159.0117 63.12) (width 0.2) (layer "F.Cu") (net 22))
 (segment (start 154.94 66.04) (end 156.0917 66.04) (width 0.2) (layer "F.Cu") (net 22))
 (segment (start 159.0117 63.12) (end 156.0917 66.04) (width 0.2) (layer "F.Cu") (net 22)))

